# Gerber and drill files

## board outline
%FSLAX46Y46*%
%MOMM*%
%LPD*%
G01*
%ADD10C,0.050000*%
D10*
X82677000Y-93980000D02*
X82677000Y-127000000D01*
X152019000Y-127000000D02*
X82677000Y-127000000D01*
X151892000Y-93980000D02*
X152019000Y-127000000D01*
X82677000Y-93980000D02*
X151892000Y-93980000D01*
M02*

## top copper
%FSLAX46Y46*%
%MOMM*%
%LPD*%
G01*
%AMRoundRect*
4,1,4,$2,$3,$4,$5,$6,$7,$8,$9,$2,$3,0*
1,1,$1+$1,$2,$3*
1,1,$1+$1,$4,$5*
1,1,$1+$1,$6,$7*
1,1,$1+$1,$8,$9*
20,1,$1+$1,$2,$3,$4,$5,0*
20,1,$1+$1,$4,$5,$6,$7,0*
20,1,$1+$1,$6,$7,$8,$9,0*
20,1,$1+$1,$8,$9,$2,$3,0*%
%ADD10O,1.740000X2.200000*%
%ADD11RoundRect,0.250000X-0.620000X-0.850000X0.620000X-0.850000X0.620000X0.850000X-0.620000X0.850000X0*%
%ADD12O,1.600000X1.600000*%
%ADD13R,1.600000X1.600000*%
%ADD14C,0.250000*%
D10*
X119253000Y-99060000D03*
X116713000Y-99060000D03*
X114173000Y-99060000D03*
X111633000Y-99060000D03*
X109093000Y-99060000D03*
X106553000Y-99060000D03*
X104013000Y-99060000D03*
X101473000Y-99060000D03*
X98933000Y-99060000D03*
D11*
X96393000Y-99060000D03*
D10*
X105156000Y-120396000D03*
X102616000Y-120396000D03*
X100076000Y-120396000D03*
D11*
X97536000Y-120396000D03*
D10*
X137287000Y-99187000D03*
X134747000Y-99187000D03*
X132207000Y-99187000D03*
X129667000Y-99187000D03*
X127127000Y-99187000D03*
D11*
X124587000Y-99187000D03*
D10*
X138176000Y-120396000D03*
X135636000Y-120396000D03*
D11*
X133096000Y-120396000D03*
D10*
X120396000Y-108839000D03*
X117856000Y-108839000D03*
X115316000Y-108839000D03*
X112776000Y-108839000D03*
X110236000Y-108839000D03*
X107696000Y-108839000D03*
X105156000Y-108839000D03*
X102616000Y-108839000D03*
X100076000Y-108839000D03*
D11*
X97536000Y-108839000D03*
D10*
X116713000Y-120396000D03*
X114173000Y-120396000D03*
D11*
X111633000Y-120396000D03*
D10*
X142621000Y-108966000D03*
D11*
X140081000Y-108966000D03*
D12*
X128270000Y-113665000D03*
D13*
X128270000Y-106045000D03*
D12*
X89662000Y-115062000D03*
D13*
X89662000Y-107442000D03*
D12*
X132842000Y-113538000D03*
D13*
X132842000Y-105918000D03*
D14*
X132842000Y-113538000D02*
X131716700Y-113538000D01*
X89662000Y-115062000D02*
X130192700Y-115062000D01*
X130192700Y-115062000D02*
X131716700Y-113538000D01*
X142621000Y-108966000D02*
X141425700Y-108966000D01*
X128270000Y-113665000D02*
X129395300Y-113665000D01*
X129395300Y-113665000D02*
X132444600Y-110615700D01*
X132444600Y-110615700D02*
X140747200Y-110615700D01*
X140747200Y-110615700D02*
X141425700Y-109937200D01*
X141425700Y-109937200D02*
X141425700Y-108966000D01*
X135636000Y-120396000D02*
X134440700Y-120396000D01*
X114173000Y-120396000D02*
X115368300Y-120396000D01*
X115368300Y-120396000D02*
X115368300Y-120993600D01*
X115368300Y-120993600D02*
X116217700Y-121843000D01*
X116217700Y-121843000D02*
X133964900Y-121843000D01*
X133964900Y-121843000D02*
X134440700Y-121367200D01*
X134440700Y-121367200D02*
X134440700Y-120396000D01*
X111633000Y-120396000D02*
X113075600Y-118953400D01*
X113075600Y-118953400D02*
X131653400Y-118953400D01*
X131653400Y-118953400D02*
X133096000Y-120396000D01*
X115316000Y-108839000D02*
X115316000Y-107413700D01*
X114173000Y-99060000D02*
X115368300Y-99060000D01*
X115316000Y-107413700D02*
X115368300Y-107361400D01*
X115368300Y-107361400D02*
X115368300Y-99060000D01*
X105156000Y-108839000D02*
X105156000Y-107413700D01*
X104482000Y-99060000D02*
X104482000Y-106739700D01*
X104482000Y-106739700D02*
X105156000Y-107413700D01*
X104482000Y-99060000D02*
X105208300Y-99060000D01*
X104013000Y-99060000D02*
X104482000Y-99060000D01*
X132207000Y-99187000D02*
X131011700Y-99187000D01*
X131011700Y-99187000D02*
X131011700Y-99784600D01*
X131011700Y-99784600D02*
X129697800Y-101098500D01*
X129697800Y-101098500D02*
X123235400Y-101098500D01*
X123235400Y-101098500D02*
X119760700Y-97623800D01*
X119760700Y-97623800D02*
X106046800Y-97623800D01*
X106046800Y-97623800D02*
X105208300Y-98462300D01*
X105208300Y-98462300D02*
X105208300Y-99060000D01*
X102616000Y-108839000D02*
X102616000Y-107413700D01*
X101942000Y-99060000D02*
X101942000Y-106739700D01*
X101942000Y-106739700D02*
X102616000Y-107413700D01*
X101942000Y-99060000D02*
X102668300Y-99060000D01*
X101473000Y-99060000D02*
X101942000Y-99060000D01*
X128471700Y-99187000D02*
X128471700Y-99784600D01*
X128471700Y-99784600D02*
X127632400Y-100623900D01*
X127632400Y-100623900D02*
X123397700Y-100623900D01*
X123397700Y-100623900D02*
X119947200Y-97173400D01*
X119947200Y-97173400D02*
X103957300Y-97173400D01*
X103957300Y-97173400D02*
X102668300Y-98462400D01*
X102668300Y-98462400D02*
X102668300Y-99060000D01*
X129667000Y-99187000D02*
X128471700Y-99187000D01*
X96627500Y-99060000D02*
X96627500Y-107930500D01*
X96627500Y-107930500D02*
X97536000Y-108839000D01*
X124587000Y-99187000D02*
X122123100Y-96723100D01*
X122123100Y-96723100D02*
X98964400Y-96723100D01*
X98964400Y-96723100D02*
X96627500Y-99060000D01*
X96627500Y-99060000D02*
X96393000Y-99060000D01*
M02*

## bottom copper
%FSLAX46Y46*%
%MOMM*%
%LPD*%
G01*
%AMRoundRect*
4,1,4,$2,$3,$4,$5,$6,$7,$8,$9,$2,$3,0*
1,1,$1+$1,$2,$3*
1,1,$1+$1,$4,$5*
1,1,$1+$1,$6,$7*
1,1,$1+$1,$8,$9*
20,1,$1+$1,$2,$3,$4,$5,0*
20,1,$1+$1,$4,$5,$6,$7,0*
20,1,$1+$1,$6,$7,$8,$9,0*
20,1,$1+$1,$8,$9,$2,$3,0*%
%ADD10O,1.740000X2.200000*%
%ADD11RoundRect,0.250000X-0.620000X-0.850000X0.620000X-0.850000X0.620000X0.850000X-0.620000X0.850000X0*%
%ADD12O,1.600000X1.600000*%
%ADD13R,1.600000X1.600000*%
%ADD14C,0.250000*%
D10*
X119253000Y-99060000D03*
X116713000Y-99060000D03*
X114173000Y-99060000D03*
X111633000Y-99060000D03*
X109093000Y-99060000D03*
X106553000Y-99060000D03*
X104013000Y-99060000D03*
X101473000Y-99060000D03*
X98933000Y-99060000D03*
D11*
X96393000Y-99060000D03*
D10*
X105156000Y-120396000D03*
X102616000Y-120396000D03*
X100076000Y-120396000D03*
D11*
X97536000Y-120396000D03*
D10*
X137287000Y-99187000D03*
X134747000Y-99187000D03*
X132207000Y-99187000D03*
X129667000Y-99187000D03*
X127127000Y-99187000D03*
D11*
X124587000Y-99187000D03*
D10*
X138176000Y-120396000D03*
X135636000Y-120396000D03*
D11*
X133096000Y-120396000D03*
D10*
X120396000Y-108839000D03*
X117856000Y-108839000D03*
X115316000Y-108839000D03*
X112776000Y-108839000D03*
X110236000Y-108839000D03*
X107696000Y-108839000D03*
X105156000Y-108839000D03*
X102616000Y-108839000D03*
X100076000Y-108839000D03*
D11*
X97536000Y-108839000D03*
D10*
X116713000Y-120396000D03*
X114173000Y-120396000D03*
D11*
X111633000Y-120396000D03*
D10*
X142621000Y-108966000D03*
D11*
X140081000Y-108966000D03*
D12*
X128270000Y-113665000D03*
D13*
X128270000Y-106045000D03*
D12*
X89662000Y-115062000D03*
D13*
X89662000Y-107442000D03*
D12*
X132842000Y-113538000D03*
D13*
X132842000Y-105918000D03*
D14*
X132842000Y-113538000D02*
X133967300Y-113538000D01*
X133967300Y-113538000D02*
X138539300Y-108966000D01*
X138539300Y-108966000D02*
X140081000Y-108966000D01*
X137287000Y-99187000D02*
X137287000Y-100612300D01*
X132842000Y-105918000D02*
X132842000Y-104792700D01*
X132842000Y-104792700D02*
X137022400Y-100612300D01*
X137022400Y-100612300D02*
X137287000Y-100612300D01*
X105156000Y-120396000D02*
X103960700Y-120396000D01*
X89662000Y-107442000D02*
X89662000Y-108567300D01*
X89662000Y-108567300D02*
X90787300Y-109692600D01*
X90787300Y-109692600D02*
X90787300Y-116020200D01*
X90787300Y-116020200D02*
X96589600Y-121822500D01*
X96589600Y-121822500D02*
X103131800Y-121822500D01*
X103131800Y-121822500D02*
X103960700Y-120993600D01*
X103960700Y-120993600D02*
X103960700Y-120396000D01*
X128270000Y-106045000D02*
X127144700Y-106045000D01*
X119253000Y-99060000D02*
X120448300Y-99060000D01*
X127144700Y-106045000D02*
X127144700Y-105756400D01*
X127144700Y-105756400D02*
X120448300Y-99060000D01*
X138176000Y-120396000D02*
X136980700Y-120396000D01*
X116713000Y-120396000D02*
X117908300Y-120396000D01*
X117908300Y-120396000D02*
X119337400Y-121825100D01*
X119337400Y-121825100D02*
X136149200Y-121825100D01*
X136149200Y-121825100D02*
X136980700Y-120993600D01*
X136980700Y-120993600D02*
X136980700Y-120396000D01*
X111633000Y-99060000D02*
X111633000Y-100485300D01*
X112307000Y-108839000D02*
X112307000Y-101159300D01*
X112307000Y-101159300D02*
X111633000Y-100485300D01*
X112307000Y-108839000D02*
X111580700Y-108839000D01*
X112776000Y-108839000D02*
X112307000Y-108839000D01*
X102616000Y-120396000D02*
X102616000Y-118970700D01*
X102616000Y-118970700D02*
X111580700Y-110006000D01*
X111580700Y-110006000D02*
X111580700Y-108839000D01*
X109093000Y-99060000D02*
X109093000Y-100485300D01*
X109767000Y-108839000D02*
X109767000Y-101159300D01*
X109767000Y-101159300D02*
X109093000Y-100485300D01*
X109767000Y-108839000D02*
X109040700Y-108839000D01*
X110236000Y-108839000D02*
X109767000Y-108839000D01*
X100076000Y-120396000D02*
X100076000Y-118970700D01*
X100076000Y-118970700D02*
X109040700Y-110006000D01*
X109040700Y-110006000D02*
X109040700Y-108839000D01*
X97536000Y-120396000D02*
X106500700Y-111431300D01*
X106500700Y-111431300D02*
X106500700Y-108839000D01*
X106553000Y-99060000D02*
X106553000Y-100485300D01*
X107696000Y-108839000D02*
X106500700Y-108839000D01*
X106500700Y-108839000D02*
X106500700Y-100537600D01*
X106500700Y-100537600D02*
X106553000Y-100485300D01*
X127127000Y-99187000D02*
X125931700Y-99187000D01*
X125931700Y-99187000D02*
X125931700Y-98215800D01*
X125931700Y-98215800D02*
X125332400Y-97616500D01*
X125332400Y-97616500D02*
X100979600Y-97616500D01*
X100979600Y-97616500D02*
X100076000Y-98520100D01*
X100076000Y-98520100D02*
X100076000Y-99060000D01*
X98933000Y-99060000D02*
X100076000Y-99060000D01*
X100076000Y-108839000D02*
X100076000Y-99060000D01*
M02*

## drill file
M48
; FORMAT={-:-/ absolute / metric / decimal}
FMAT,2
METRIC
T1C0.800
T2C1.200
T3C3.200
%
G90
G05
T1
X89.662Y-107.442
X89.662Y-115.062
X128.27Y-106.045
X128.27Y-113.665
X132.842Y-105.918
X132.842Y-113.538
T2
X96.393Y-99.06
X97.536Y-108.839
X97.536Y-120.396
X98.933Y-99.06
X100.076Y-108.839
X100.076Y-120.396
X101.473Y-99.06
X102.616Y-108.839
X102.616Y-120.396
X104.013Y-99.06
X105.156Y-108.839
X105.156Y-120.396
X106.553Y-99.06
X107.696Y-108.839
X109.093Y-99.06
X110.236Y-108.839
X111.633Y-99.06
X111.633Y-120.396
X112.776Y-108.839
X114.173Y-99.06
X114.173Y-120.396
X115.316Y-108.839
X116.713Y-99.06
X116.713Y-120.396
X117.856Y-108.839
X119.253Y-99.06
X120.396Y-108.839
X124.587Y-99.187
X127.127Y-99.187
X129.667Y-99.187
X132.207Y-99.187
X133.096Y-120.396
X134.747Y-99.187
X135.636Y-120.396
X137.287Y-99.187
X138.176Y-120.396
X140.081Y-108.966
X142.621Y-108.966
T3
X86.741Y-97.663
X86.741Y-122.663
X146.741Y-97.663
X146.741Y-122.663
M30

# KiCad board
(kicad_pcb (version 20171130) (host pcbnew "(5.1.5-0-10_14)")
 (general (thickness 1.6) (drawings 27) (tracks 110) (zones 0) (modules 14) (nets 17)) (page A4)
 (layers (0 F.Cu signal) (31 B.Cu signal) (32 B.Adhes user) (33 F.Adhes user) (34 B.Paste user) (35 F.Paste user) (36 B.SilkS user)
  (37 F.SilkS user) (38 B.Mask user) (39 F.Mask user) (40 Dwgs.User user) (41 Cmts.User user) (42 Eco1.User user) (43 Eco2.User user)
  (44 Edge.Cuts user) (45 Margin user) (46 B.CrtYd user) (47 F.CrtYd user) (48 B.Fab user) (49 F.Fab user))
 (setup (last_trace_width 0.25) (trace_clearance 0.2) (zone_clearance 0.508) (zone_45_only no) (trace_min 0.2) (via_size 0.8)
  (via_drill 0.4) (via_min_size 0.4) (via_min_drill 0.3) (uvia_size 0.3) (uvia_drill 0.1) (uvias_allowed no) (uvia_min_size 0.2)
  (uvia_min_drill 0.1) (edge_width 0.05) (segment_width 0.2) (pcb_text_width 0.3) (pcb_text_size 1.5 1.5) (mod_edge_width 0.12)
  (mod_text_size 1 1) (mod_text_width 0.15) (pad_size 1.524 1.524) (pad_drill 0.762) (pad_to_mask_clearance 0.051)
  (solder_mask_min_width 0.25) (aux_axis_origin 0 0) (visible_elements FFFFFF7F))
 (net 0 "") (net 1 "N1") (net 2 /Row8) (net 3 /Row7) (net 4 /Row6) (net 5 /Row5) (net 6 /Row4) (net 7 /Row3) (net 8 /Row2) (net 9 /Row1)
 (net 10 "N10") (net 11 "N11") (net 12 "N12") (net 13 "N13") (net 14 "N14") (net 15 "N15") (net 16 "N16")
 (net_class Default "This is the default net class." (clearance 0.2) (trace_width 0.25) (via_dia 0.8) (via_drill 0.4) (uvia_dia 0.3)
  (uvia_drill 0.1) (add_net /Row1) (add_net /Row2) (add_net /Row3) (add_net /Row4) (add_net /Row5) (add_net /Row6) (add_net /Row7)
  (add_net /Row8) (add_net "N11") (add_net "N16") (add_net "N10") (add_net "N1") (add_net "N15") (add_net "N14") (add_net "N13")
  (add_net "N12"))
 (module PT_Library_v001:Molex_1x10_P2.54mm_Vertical (layer F.Cu) (at 96.393 99.06)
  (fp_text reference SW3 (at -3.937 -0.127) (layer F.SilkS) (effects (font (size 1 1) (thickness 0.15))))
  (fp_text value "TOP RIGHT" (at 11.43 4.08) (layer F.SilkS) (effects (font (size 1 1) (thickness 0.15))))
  (pad 10 thru_hole oval (at 22.86 0) (size 1.74 2.2) (drill 1.2) (layers *.Cu *.Mask) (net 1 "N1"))
  (pad 9 thru_hole oval (at 20.32 0) (size 1.74 2.2) (drill 1.2) (layers *.Cu *.Mask))
  (pad 8 thru_hole oval (at 17.78 0) (size 1.74 2.2) (drill 1.2) (layers *.Cu *.Mask) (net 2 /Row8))
  (pad 7 thru_hole oval (at 15.24 0) (size 1.74 2.2) (drill 1.2) (layers *.Cu *.Mask) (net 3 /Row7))
  (pad 6 thru_hole oval (at 12.7 0) (size 1.74 2.2) (drill 1.2) (layers *.Cu *.Mask) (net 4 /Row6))
  (pad 5 thru_hole oval (at 10.16 0) (size 1.74 2.2) (drill 1.2) (layers *.Cu *.Mask) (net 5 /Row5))
  (pad 4 thru_hole oval (at 7.62 0) (size 1.74 2.2) (drill 1.2) (layers *.Cu *.Mask) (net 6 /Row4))
  (pad 3 thru_hole oval (at 5.08 0) (size 1.74 2.2) (drill 1.2) (layers *.Cu *.Mask) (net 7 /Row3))
  (pad 2 thru_hole oval (at 2.54 0) (size 1.74 2.2) (drill 1.2) (layers *.Cu *.Mask) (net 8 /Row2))
  (pad 1 thru_hole roundrect (at 0 0) (size 1.74 2.2) (drill 1.2) (layers *.Cu *.Mask) (roundrect_rratio 0.143678) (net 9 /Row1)))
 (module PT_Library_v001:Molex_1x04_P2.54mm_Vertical (layer F.Cu) (at 97.536 120.396)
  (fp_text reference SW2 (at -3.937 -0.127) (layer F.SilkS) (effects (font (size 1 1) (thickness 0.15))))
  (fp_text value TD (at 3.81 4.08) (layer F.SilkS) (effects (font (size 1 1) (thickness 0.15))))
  (pad 4 thru_hole oval (at 7.62 0) (size 1.74 2.2) (drill 1.2) (layers *.Cu *.Mask) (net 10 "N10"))
  (pad 3 thru_hole oval (at 5.08 0) (size 1.74 2.2) (drill 1.2) (layers *.Cu *.Mask) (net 3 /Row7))
  (pad 2 thru_hole oval (at 2.54 0) (size 1.74 2.2) (drill 1.2) (layers *.Cu *.Mask) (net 4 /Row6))
  (pad 1 thru_hole roundrect (at 0 0) (size 1.74 2.2) (drill 1.2) (layers *.Cu *.Mask) (roundrect_rratio 0.143678) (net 5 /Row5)))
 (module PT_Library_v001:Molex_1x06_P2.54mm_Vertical (layer F.Cu) (at 124.587 99.187)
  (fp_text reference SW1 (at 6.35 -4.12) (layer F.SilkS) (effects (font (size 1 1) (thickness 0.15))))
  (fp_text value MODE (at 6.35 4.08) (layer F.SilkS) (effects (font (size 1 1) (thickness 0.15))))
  (pad 6 thru_hole oval (at 12.7 0) (size 1.74 2.2) (drill 1.2) (layers *.Cu *.Mask) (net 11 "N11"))
  (pad 5 thru_hole oval (at 10.16 0) (size 1.74 2.2) (drill 1.2) (layers *.Cu *.Mask))
  (pad 4 thru_hole oval (at 7.62 0) (size 1.74 2.2) (drill 1.2) (layers *.Cu *.Mask) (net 6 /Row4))
  (pad 3 thru_hole oval (at 5.08 0) (size 1.74 2.2) (drill 1.2) (layers *.Cu *.Mask) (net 7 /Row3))
  (pad 2 thru_hole oval (at 2.54 0) (size 1.74 2.2) (drill 1.2) (layers *.Cu *.Mask) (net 8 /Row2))
  (pad 1 thru_hole roundrect (at 0 0) (size 1.74 2.2) (drill 1.2) (layers *.Cu *.Mask) (roundrect_rratio 0.143678) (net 9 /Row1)))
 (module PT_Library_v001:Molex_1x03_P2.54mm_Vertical (layer F.Cu) (at 133.096 120.396)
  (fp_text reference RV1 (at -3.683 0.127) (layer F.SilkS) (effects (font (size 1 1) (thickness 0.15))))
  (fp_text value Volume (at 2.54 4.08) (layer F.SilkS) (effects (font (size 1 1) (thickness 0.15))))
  (pad 3 thru_hole oval (at 5.08 0) (size 1.74 2.2) (drill 1.2) (layers *.Cu *.Mask) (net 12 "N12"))
  (pad 2 thru_hole oval (at 2.54 0) (size 1.74 2.2) (drill 1.2) (layers *.Cu *.Mask) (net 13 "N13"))
  (pad 1 thru_hole roundrect (at 0 0) (size 1.74 2.2) (drill 1.2) (layers *.Cu *.Mask) (roundrect_rratio 0.143678) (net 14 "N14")))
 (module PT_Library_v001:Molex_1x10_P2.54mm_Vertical (layer F.Cu) (at 97.536 108.839)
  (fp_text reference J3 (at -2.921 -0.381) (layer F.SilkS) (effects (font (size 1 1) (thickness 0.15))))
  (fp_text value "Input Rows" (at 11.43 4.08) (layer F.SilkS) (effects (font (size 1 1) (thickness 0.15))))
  (pad 10 thru_hole oval (at 22.86 0) (size 1.74 2.2) (drill 1.2) (layers *.Cu *.Mask))
  (pad 9 thru_hole oval (at 20.32 0) (size 1.74 2.2) (drill 1.2) (layers *.Cu *.Mask))
  (pad 8 thru_hole oval (at 17.78 0) (size 1.74 2.2) (drill 1.2) (layers *.Cu *.Mask) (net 2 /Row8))
  (pad 7 thru_hole oval (at 15.24 0) (size 1.74 2.2) (drill 1.2) (layers *.Cu *.Mask) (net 3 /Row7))
  (pad 6 thru_hole oval (at 12.7 0) (size 1.74 2.2) (drill 1.2) (layers *.Cu *.Mask) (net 4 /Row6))
  (pad 5 thru_hole oval (at 10.16 0) (size 1.74 2.2) (drill 1.2) (layers *.Cu *.Mask) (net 5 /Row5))
  (pad 4 thru_hole oval (at 7.62 0) (size 1.74 2.2) (drill 1.2) (layers *.Cu *.Mask) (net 6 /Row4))
  (pad 3 thru_hole oval (at 5.08 0) (size 1.74 2.2) (drill 1.2) (layers *.Cu *.Mask) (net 7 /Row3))
  (pad 2 thru_hole oval (at 2.54 0) (size 1.74 2.2) (drill 1.2) (layers *.Cu *.Mask) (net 8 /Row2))
  (pad 1 thru_hole roundrect (at 0 0) (size 1.74 2.2) (drill 1.2) (layers *.Cu *.Mask) (roundrect_rratio 0.143678) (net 9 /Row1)))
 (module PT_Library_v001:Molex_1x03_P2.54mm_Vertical (layer F.Cu) (at 111.633 120.396)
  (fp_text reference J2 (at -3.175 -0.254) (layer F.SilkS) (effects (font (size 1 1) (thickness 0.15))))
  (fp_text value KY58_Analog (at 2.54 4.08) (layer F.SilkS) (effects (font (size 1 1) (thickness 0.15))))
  (pad 3 thru_hole oval (at 5.08 0) (size 1.74 2.2) (drill 1.2) (layers *.Cu *.Mask) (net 12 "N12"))
  (pad 2 thru_hole oval (at 2.54 0) (size 1.74 2.2) (drill 1.2) (layers *.Cu *.Mask) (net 13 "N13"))
  (pad 1 thru_hole roundrect (at 0 0) (size 1.74 2.2) (drill 1.2) (layers *.Cu *.Mask) (roundrect_rratio 0.143678) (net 14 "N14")))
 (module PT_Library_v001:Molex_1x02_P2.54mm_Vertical (layer F.Cu) (at 140.081 108.966)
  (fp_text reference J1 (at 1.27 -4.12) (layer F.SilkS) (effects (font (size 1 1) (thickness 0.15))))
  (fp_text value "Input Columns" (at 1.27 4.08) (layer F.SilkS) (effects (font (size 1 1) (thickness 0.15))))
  (pad 2 thru_hole oval (at 2.54 0) (size 1.74 2.2) (drill 1.2) (layers *.Cu *.Mask) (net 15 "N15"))
  (pad 1 thru_hole roundrect (at 0 0) (size 1.74 2.2) (drill 1.2) (layers *.Cu *.Mask) (roundrect_rratio 0.143678) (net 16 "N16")))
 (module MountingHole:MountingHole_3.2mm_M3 (layer F.Cu) (at 86.741 97.663)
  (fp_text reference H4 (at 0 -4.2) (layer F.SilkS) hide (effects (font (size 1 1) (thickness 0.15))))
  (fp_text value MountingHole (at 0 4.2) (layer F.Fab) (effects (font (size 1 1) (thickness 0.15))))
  (pad 1 np_thru_hole circle (at 0 0) (size 3.2 3.2) (drill 3.2) (layers *.Cu *.Mask)))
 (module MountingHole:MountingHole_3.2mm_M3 (layer F.Cu) (at 86.741 122.663)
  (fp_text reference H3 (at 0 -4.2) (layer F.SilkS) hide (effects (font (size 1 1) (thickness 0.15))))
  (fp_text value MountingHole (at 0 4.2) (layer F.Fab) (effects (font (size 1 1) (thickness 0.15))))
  (pad 1 np_thru_hole circle (at 0 0) (size 3.2 3.2) (drill 3.2) (layers *.Cu *.Mask)))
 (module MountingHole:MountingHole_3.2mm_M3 (layer F.Cu) (at 146.741 97.663)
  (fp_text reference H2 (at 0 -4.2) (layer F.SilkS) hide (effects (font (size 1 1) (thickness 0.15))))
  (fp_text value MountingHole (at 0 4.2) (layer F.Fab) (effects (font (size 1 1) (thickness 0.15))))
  (pad 1 np_thru_hole circle (at 0 0) (size 3.2 3.2) (drill 3.2) (layers *.Cu *.Mask)))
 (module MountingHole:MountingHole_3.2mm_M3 (layer F.Cu) (at 146.741 122.663)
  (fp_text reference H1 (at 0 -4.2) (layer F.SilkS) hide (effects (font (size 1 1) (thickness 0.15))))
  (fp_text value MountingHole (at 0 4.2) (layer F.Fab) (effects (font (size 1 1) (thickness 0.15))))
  (pad 1 np_thru_hole circle (at 0 0) (size 3.2 3.2) (drill 3.2) (layers *.Cu *.Mask)))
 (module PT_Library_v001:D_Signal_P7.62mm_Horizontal (layer F.Cu) (at 128.27 106.045 270)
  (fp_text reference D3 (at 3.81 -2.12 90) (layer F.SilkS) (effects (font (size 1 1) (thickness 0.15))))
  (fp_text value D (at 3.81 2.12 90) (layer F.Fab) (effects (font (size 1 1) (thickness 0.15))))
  (pad 2 thru_hole oval (at 7.62 0 270) (size 1.6 1.6) (drill 0.8) (layers *.Cu *.Mask) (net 15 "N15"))
  (pad 1 thru_hole rect (at 0 0 270) (size 1.6 1.6) (drill 0.8) (layers *.Cu *.Mask) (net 1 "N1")))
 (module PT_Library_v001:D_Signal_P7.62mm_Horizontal (layer F.Cu) (at 89.662 107.442 270)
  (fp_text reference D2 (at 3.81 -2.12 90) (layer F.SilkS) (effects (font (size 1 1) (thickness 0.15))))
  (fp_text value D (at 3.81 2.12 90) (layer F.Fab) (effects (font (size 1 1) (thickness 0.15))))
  (pad 2 thru_hole oval (at 7.62 0 270) (size 1.6 1.6) (drill 0.8) (layers *.Cu *.Mask) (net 16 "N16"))
  (pad 1 thru_hole rect (at 0 0 270) (size 1.6 1.6) (drill 0.8) (layers *.Cu *.Mask) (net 10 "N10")))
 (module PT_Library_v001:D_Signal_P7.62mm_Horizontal (layer F.Cu) (at 132.842 105.918 270)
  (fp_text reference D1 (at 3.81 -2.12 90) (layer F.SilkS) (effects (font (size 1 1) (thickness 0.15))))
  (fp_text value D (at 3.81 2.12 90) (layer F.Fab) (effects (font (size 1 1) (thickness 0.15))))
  (pad 2 thru_hole oval (at 7.62 0 270) (size 1.6 1.6) (drill 0.8) (layers *.Cu *.Mask) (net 16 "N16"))
  (pad 1 thru_hole rect (at 0 0 270) (size 1.6 1.6) (drill 0.8) (layers *.Cu *.Mask) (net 11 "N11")))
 (gr_line (start 82.677 93.98) (end 82.677 127) (layer Edge.Cuts) (width 0.05))
 (gr_line (start 152.019 127) (end 82.677 127) (layer Edge.Cuts) (width 0.05))
 (gr_line (start 151.892 93.98) (end 152.019 127) (layer Edge.Cuts) (width 0.05))
 (gr_line (start 82.677 93.98) (end 151.892 93.98) (layer Edge.Cuts) (width 0.05))
 (segment (start 132.842 113.538) (end 131.7167 113.538) (width 0.25) (layer F.Cu) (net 16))
 (segment (start 89.662 115.062) (end 130.1927 115.062) (width 0.25) (layer F.Cu) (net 16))
 (segment (start 130.1927 115.062) (end 131.7167 113.538) (width 0.25) (layer F.Cu) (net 16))
 (segment (start 132.842 113.538) (end 133.9673 113.538) (width 0.25) (layer B.Cu) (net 16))
 (segment (start 133.9673 113.538) (end 138.5393 108.966) (width 0.25) (layer B.Cu) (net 16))
 (segment (start 138.5393 108.966) (end 140.081 108.966) (width 0.25) (layer B.Cu) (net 16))
 (segment (start 137.287 99.187) (end 137.287 100.6123) (width 0.25) (layer B.Cu) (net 11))
 (segment (start 132.842 105.918) (end 132.842 104.7927) (width 0.25) (layer B.Cu) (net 11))
 (segment (start 132.842 104.7927) (end 137.0224 100.6123) (width 0.25) (layer B.Cu) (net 11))
 (segment (start 137.0224 100.6123) (end 137.287 100.6123) (width 0.25) (layer B.Cu) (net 11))
 (segment (start 105.156 120.396) (end 103.9607 120.396) (width 0.25) (layer B.Cu) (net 10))
 (segment (start 89.662 107.442) (end 89.662 108.5673) (width 0.25) (layer B.Cu) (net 10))
 (segment (start 89.662 108.5673) (end 90.7873 109.6926) (width 0.25) (layer B.Cu) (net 10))
 (segment (start 90.7873 109.6926) (end 90.7873 116.0202) (width 0.25) (layer B.Cu) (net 10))
 (segment (start 90.7873 116.0202) (end 96.5896 121.8225) (width 0.25) (layer B.Cu) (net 10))
 (segment (start 96.5896 121.8225) (end 103.1318 121.8225) (width 0.25) (layer B.Cu) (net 10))
 (segment (start 103.1318 121.8225) (end 103.9607 120.9936) (width 0.25) (layer B.Cu) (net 10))
 (segment (start 103.9607 120.9936) (end 103.9607 120.396) (width 0.25) (layer B.Cu) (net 10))
 (segment (start 142.621 108.966) (end 141.4257 108.966) (width 0.25) (layer F.Cu) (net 15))
 (segment (start 128.27 113.665) (end 129.3953 113.665) (width 0.25) (layer F.Cu) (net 15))
 (segment (start 129.3953 113.665) (end 132.4446 110.6157) (width 0.25) (layer F.Cu) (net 15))
 (segment (start 132.4446 110.6157) (end 140.7472 110.6157) (width 0.25) (layer F.Cu) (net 15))
 (segment (start 140.7472 110.6157) (end 141.4257 109.9372) (width 0.25) (layer F.Cu) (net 15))
 (segment (start 141.4257 109.9372) (end 141.4257 108.966) (width 0.25) (layer F.Cu) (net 15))
 (segment (start 128.27 106.045) (end 127.1447 106.045) (width 0.25) (layer B.Cu) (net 1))
 (segment (start 119.253 99.06) (end 120.4483 99.06) (width 0.25) (layer B.Cu) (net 1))
 (segment (start 127.1447 106.045) (end 127.1447 105.7564) (width 0.25) (layer B.Cu) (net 1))
 (segment (start 127.1447 105.7564) (end 120.4483 99.06) (width 0.25) (layer B.Cu) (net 1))
 (segment (start 138.176 120.396) (end 136.9807 120.396) (width 0.25) (layer B.Cu) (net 12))
 (segment (start 116.713 120.396) (end 117.9083 120.396) (width 0.25) (layer B.Cu) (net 12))
 (segment (start 117.9083 120.396) (end 119.3374 121.8251) (width 0.25) (layer B.Cu) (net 12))
 (segment (start 119.3374 121.8251) (end 136.1492 121.8251) (width 0.25) (layer B.Cu) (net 12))
 (segment (start 136.1492 121.8251) (end 136.9807 120.9936) (width 0.25) (layer B.Cu) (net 12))
 (segment (start 136.9807 120.9936) (end 136.9807 120.396) (width 0.25) (layer B.Cu) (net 12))
 (segment (start 135.636 120.396) (end 134.4407 120.396) (width 0.25) (layer F.Cu) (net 13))
 (segment (start 114.173 120.396) (end 115.3683 120.396) (width 0.25) (layer F.Cu) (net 13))
 (segment (start 115.3683 120.396) (end 115.3683 120.9936) (width 0.25) (layer F.Cu) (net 13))
 (segment (start 115.3683 120.9936) (end 116.2177 121.843) (width 0.25) (layer F.Cu) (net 13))
 (segment (start 116.2177 121.843) (end 133.9649 121.843) (width 0.25) (layer F.Cu) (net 13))
 (segment (start 133.9649 121.843) (end 134.4407 121.3672) (width 0.25) (layer F.Cu) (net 13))
 (segment (start 134.4407 121.3672) (end 134.4407 120.396) (width 0.25) (layer F.Cu) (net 13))
 (segment (start 111.633 120.396) (end 113.0756 118.9534) (width 0.25) (layer F.Cu) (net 14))
 (segment (start 113.0756 118.9534) (end 131.6534 118.9534) (width 0.25) (layer F.Cu) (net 14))
 (segment (start 131.6534 118.9534) (end 133.096 120.396) (width 0.25) (layer F.Cu) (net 14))
 (segment (start 115.316 108.839) (end 115.316 107.4137) (width 0.25) (layer F.Cu) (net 2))
 (segment (start 114.173 99.06) (end 115.3683 99.06) (width 0.25) (layer F.Cu) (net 2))
 (segment (start 115.316 107.4137) (end 115.3683 107.3614) (width 0.25) (layer F.Cu) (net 2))
 (segment (start 115.3683 107.3614) (end 115.3683 99.06) (width 0.25) (layer F.Cu) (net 2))
 (segment (start 111.633 99.06) (end 111.633 100.4853) (width 0.25) (layer B.Cu) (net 3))
 (segment (start 112.307 108.839) (end 112.307 101.1593) (width 0.25) (layer B.Cu) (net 3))
 (segment (start 112.307 101.1593) (end 111.633 100.4853) (width 0.25) (layer B.Cu) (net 3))
 (segment (start 112.307 108.839) (end 111.5807 108.839) (width 0.25) (layer B.Cu) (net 3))
 (segment (start 112.776 108.839) (end 112.307 108.839) (width 0.25) (layer B.Cu) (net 3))
 (segment (start 102.616 120.396) (end 102.616 118.9707) (width 0.25) (layer B.Cu) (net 3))
 (segment (start 102.616 118.9707) (end 111.5807 110.006) (width 0.25) (layer B.Cu) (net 3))
 (segment (start 111.5807 110.006) (end 111.5807 108.839) (width 0.25) (layer B.Cu) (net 3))
 (segment (start 109.093 99.06) (end 109.093 100.4853) (width 0.25) (layer B.Cu) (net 4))
 (segment (start 109.767 108.839) (end 109.767 101.1593) (width 0.25) (layer B.Cu) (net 4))
 (segment (start 109.767 101.1593) (end 109.093 100.4853) (width 0.25) (layer B.Cu) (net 4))
 (segment (start 109.767 108.839) (end 109.0407 108.839) (width 0.25) (layer B.Cu) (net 4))
 (segment (start 110.236 108.839) (end 109.767 108.839) (width 0.25) (layer B.Cu) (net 4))
 (segment (start 100.076 120.396) (end 100.076 118.9707) (width 0.25) (layer B.Cu) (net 4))
 (segment (start 100.076 118.9707) (end 109.0407 110.006) (width 0.25) (layer B.Cu) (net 4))
 (segment (start 109.0407 110.006) (end 109.0407 108.839) (width 0.25) (layer B.Cu) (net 4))
 (segment (start 97.536 120.396) (end 106.5007 111.4313) (width 0.25) (layer B.Cu) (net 5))
 (segment (start 106.5007 111.4313) (end 106.5007 108.839) (width 0.25) (layer B.Cu) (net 5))
 (segment (start 106.553 99.06) (end 106.553 100.4853) (width 0.25) (layer B.Cu) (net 5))
 (segment (start 107.696 108.839) (end 106.5007 108.839) (width 0.25) (layer B.Cu) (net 5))
 (segment (start 106.5007 108.839) (end 106.5007 100.5376) (width 0.25) (layer B.Cu) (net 5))
 (segment (start 106.5007 100.5376) (end 106.553 100.4853) (width 0.25) (layer B.Cu) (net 5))
 (segment (start 105.156 108.839) (end 105.156 107.4137) (width 0.25) (layer F.Cu) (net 6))
 (segment (start 104.482 99.06) (end 104.482 106.7397) (width 0.25) (layer F.Cu) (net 6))
 (segment (start 104.482 106.7397) (end 105.156 107.4137) (width 0.25) (layer F.Cu) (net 6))
 (segment (start 104.482 99.06) (end 105.2083 99.06) (width 0.25) (layer F.Cu) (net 6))
 (segment (start 104.013 99.06) (end 104.482 99.06) (width 0.25) (layer F.Cu) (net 6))
 (segment (start 132.207 99.187) (end 131.0117 99.187) (width 0.25) (layer F.Cu) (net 6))
 (segment (start 131.0117 99.187) (end 131.0117 99.7846) (width 0.25) (layer F.Cu) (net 6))
 (segment (start 131.0117 99.7846) (end 129.6978 101.0985) (width 0.25) (layer F.Cu) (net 6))
 (segment (start 129.6978 101.0985) (end 123.2354 101.0985) (width 0.25) (layer F.Cu) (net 6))
 (segment (start 123.2354 101.0985) (end 119.7607 97.6238) (width 0.25) (layer F.Cu) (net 6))
 (segment (start 119.7607 97.6238) (end 106.0468 97.6238) (width 0.25) (layer F.Cu) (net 6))
 (segment (start 106.0468 97.6238) (end 105.2083 98.4623) (width 0.25) (layer F.Cu) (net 6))
 (segment (start 105.2083 98.4623) (end 105.2083 99.06) (width 0.25) (layer F.Cu) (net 6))
 (segment (start 102.616 108.839) (end 102.616 107.4137) (width 0.25) (layer F.Cu) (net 7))
 (segment (start 101.942 99.06) (end 101.942 106.7397) (width 0.25) (layer F.Cu) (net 7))
 (segment (start 101.942 106.7397) (end 102.616 107.4137) (width 0.25) (layer F.Cu) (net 7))
 (segment (start 101.942 99.06) (end 102.6683 99.06) (width 0.25) (layer F.Cu) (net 7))
 (segment (start 101.473 99.06) (end 101.942 99.06) (width 0.25) (layer F.Cu) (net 7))
 (segment (start 128.4717 99.187) (end 128.4717 99.7846) (width 0.25) (layer F.Cu) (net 7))
 (segment (start 128.4717 99.7846) (end 127.6324 100.6239) (width 0.25) (layer F.Cu) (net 7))
 (segment (start 127.6324 100.6239) (end 123.3977 100.6239) (width 0.25) (layer F.Cu) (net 7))
 (segment (start 123.3977 100.6239) (end 119.9472 97.1734) (width 0.25) (layer F.Cu) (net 7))
 (segment (start 119.9472 97.1734) (end 103.9573 97.1734) (width 0.25) (layer F.Cu) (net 7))
 (segment (start 103.9573 97.1734) (end 102.6683 98.4624) (width 0.25) (layer F.Cu) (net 7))
 (segment (start 102.6683 98.4624) (end 102.6683 99.06) (width 0.25) (layer F.Cu) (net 7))
 (segment (start 129.667 99.187) (end 128.4717 99.187) (width 0.25) (layer F.Cu) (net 7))
 (segment (start 127.127 99.187) (end 125.9317 99.187) (width 0.25) (layer B.Cu) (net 8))
 (segment (start 125.9317 99.187) (end 125.9317 98.2158) (width 0.25) (layer B.Cu) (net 8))
 (segment (start 125.9317 98.2158) (end 125.3324 97.6165) (width 0.25) (layer B.Cu) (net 8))
 (segment (start 125.3324 97.6165) (end 100.9796 97.6165) (width 0.25) (layer B.Cu) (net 8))
 (segment (start 100.9796 97.6165) (end 100.076 98.5201) (width 0.25) (layer B.Cu) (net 8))
 (segment (start 100.076 98.5201) (end 100.076 99.06) (width 0.25) (layer B.Cu) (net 8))
 (segment (start 98.933 99.06) (end 100.076 99.06) (width 0.25) (layer B.Cu) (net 8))
 (segment (start 100.076 108.839) (end 100.076 99.06) (width 0.25) (layer B.Cu) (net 8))
 (segment (start 96.6275 99.06) (end 96.6275 107.9305) (width 0.25) (layer F.Cu) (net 9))
 (segment (start 96.6275 107.9305) (end 97.536 108.839) (width 0.25) (layer F.Cu) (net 9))
 (segment (start 124.587 99.187) (end 122.1231 96.7231) (width 0.25) (layer F.Cu) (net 9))
 (segment (start 122.1231 96.7231) (end 98.9644 96.7231) (width 0.25) (layer F.Cu) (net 9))
 (segment (start 98.9644 96.7231) (end 96.6275 99.06) (width 0.25) (layer F.Cu) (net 9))
 (segment (start 96.6275 99.06) (end 96.393 99.06) (width 0.25) (layer F.Cu) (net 9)))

